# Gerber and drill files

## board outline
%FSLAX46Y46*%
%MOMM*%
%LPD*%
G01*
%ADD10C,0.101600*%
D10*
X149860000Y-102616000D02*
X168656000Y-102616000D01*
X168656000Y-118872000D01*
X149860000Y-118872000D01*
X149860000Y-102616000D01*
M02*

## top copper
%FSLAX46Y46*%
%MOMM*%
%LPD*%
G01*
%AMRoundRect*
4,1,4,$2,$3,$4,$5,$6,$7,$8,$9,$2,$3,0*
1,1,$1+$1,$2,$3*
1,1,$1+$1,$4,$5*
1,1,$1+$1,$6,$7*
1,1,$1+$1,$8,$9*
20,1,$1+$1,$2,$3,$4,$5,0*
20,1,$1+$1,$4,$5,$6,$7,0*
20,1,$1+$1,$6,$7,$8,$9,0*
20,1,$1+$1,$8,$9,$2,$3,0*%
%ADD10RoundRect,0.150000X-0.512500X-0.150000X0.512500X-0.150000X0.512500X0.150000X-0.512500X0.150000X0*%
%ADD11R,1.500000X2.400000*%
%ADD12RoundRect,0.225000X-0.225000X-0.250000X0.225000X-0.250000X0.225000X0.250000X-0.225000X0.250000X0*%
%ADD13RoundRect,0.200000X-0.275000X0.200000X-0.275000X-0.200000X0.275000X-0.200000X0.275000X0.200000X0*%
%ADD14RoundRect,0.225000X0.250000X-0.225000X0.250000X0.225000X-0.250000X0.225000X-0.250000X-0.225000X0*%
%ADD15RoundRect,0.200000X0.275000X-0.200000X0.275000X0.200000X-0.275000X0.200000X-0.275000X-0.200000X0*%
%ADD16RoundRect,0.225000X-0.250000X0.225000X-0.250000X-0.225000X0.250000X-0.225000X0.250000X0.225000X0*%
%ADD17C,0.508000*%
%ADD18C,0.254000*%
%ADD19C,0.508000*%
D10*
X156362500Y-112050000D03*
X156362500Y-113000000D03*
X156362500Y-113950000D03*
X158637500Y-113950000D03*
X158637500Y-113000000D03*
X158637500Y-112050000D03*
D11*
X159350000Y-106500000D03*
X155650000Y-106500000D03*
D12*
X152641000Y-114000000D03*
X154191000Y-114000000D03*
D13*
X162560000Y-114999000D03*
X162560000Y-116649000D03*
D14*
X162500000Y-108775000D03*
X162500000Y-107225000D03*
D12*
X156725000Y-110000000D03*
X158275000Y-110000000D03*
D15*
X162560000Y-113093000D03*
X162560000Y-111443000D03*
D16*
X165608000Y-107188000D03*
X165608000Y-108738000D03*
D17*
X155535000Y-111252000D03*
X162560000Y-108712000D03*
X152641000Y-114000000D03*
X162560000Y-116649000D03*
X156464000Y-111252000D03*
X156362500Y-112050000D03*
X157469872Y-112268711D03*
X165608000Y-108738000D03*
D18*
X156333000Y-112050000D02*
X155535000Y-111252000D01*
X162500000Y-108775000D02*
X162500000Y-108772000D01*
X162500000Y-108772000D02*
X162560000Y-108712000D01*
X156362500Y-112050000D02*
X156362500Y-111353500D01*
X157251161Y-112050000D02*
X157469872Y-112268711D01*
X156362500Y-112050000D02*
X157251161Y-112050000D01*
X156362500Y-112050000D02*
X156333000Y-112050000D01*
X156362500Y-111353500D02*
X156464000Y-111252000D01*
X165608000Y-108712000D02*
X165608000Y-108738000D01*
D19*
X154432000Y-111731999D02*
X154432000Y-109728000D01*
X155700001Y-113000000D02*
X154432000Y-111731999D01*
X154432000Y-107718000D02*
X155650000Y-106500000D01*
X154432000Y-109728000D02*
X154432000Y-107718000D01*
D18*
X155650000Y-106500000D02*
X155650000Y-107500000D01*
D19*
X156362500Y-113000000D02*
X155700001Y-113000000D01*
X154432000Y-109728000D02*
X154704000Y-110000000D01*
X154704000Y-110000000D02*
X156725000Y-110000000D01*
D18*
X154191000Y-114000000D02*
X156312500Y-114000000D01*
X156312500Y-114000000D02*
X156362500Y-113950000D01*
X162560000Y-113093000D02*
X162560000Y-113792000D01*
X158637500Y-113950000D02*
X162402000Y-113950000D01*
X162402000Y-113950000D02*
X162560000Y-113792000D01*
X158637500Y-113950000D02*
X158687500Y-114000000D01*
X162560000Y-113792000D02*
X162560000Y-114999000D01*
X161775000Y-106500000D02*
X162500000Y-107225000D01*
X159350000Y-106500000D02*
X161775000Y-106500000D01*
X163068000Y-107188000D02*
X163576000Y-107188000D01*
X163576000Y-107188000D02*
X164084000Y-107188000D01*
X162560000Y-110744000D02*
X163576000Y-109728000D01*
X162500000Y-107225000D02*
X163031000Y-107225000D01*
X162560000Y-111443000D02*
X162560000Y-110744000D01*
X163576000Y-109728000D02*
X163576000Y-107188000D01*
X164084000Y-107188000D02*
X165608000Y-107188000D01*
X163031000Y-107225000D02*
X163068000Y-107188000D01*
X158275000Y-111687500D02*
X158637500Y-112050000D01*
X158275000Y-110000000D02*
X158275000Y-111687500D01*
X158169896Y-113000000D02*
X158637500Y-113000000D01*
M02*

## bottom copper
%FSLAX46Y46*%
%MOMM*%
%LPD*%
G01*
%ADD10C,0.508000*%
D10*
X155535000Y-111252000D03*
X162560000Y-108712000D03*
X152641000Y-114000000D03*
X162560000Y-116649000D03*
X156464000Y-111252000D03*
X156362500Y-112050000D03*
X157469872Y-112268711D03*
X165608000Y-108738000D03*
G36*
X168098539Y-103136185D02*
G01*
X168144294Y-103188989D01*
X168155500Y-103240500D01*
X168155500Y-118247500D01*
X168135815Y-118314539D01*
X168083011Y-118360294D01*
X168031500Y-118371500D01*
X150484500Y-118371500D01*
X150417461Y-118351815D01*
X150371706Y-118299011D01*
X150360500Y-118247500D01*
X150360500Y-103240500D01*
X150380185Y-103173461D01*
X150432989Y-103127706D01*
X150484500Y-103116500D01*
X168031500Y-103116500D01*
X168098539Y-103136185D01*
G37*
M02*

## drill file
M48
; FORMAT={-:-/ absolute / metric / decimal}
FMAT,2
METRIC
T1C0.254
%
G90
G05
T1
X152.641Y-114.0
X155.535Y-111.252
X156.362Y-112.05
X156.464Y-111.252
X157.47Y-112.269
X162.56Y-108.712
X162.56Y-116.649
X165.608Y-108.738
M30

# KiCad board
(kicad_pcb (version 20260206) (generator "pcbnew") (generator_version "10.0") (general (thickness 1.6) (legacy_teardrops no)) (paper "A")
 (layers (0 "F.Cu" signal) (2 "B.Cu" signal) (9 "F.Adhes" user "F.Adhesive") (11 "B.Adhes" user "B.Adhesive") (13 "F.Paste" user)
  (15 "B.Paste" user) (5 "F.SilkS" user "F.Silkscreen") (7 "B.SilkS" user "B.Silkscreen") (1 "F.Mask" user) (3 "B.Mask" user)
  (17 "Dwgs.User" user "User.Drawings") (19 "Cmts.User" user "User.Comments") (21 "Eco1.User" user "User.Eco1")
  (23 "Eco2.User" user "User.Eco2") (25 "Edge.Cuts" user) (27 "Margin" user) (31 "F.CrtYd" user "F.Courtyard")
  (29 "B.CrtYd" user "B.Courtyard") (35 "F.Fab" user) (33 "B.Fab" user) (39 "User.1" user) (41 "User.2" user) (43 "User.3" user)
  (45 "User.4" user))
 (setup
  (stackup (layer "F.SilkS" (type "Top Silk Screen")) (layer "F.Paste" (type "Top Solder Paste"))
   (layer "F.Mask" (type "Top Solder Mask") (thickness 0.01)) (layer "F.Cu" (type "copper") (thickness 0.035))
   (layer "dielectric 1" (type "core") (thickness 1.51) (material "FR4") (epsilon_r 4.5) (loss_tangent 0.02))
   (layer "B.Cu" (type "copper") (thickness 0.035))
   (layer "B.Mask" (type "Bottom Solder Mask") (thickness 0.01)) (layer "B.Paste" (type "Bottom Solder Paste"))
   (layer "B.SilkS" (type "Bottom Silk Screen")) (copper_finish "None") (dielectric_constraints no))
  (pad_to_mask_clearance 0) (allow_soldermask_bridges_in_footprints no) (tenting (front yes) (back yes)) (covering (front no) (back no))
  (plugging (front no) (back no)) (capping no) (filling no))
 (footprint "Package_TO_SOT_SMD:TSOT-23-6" (layer "F.Cu") (at 157.5 113)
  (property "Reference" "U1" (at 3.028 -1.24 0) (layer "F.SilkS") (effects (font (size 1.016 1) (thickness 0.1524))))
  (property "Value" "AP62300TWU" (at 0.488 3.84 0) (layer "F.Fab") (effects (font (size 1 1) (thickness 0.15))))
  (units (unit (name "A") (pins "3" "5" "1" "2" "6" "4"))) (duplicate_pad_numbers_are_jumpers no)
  (pad "1" smd roundrect (at -1.1375 -0.95) (size 1.325 0.6) (layers "F.Cu" "F.Mask" "F.Paste") (roundrect_rratio 0.25) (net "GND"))
  (pad "2" smd roundrect (at -1.1375 0) (size 1.325 0.6) (layers "F.Cu" "F.Mask" "F.Paste") (roundrect_rratio 0.25) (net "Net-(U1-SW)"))
  (pad "3" smd roundrect (at -1.1375 0.95) (size 1.325 0.6) (layers "F.Cu" "F.Mask" "F.Paste") (roundrect_rratio 0.25) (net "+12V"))
  (pad "4" smd roundrect (at 1.1375 0.95) (size 1.325 0.6) (layers "F.Cu" "F.Mask" "F.Paste") (roundrect_rratio 0.25) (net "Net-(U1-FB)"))
  (pad "5" smd roundrect (at 1.1375 0) (size 1.325 0.6) (layers "F.Cu" "F.Mask" "F.Paste") (roundrect_rratio 0.25)
   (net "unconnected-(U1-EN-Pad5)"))
  (pad "6" smd roundrect (at 1.1375 -0.95) (size 1.325 0.6) (layers "F.Cu" "F.Mask" "F.Paste") (roundrect_rratio 0.25) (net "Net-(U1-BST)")))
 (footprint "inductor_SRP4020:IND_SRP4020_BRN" (layer "F.Cu") (at 157.5 106.5 180)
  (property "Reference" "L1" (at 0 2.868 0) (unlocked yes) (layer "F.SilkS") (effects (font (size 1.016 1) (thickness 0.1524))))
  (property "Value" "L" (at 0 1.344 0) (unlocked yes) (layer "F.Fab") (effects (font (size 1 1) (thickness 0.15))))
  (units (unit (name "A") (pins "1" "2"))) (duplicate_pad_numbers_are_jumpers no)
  (pad "1" smd rect (at -1.85 0 270) (size 2.4 1.5) (layers "F.Cu" "F.Mask" "F.Paste") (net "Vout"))
  (pad "2" smd rect (at 1.85 0 270) (size 2.4 1.5) (layers "F.Cu" "F.Mask" "F.Paste") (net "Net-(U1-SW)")))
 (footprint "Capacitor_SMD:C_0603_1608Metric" (layer "F.Cu") (at 153.416 114)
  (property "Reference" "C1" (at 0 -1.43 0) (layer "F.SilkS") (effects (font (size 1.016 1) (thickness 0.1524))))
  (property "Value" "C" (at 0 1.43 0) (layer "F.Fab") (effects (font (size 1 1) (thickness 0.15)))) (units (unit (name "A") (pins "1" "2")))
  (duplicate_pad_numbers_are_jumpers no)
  (pad "1" smd roundrect (at -0.775 0) (size 0.9 0.95) (layers "F.Cu" "F.Mask" "F.Paste") (roundrect_rratio 0.25) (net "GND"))
  (pad "2" smd roundrect (at 0.775 0) (size 0.9 0.95) (layers "F.Cu" "F.Mask" "F.Paste") (roundrect_rratio 0.25) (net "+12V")))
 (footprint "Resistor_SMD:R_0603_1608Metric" (layer "F.Cu") (at 162.56 115.824 -90)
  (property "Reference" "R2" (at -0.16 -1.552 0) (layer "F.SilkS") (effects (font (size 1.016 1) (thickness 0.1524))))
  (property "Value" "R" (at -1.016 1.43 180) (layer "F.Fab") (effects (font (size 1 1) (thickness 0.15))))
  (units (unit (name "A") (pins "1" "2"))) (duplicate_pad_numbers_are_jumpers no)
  (pad "1" smd roundrect (at -0.825 0 270) (size 0.8 0.95) (layers "F.Cu" "F.Mask" "F.Paste") (roundrect_rratio 0.25) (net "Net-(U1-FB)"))
  (pad "2" smd roundrect (at 0.825 0 270) (size 0.8 0.95) (layers "F.Cu" "F.Mask" "F.Paste") (roundrect_rratio 0.25) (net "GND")))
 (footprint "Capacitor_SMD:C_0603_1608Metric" (layer "F.Cu") (at 162.5 108 90)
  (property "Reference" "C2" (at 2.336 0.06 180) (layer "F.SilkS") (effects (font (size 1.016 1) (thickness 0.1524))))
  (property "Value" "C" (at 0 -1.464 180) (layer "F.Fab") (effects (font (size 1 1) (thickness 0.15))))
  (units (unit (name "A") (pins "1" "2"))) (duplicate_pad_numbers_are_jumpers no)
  (pad "1" smd roundrect (at -0.775 0 90) (size 0.9 0.95) (layers "F.Cu" "F.Mask" "F.Paste") (roundrect_rratio 0.25) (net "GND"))
  (pad "2" smd roundrect (at 0.775 0 90) (size 0.9 0.95) (layers "F.Cu" "F.Mask" "F.Paste") (roundrect_rratio 0.25) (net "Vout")))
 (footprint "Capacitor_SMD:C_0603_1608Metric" (layer "F.Cu") (at 157.5 110)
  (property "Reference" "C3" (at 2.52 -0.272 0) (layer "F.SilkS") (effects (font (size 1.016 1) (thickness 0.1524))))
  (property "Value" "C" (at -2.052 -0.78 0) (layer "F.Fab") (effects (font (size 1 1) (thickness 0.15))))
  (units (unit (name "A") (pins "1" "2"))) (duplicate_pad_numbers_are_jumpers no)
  (pad "1" smd roundrect (at -0.775 0) (size 0.9 0.95) (layers "F.Cu" "F.Mask" "F.Paste") (roundrect_rratio 0.25) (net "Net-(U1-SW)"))
  (pad "2" smd roundrect (at 0.775 0) (size 0.9 0.95) (layers "F.Cu" "F.Mask" "F.Paste") (roundrect_rratio 0.25) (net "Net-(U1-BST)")))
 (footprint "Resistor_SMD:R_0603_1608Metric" (layer "F.Cu") (at 162.56 112.268 90)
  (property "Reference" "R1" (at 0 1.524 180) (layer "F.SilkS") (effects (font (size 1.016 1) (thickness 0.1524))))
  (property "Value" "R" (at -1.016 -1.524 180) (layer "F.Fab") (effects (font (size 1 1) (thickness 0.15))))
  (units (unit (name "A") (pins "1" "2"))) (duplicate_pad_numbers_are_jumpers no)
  (pad "1" smd roundrect (at -0.825 0 90) (size 0.8 0.95) (layers "F.Cu" "F.Mask" "F.Paste") (roundrect_rratio 0.25) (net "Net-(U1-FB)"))
  (pad "2" smd roundrect (at 0.825 0 90) (size 0.8 0.95) (layers "F.Cu" "F.Mask" "F.Paste") (roundrect_rratio 0.25) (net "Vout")))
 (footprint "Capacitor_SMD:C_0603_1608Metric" (layer "F.Cu") (at 165.608 107.963 -90)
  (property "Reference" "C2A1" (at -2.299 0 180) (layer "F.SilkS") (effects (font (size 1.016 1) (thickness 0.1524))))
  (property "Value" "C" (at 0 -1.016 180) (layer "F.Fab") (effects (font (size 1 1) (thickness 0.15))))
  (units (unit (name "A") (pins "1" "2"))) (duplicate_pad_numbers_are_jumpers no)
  (pad "1" smd roundrect (at -0.775 0 270) (size 0.9 0.95) (layers "F.Cu" "F.Mask" "F.Paste") (roundrect_rratio 0.25) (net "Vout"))
  (pad "2" smd roundrect (at 0.775 0 270) (size 0.9 0.95) (layers "F.Cu" "F.Mask" "F.Paste") (roundrect_rratio 0.25) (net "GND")))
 (gr_rect (start 149.86 102.616) (end 168.656 118.872) (stroke (width 0.1016) (type default)) (fill no) (layer "Edge.Cuts"))
 (segment (start 156.333 112.05) (end 155.535 111.252) (width 0.254) (layer "F.Cu") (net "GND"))
 (segment (start 162.5 108.775) (end 162.5 108.772) (width 0.254) (layer "F.Cu") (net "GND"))
 (segment (start 162.5 108.772) (end 162.56 108.712) (width 0.254) (layer "F.Cu") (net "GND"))
 (segment (start 156.3625 112.05) (end 156.3625 111.3535) (width 0.254) (layer "F.Cu") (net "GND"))
 (segment (start 157.251161 112.05) (end 157.469872 112.268711) (width 0.254) (layer "F.Cu") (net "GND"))
 (segment (start 156.3625 112.05) (end 157.251161 112.05) (width 0.254) (layer "F.Cu") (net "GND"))
 (segment (start 156.3625 112.05) (end 156.333 112.05) (width 0.254) (layer "F.Cu") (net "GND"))
 (segment (start 156.3625 111.3535) (end 156.464 111.252) (width 0.254) (layer "F.Cu") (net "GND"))
 (segment (start 165.608 108.712) (end 165.608 108.738) (width 0.254) (layer "F.Cu") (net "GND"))
 (via (at 155.535 111.252) (size 0.508) (drill 0.254) (layers "F.Cu" "B.Cu") (free yes) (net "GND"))
 (via (at 162.56 108.712) (size 0.508) (drill 0.254) (layers "F.Cu" "B.Cu") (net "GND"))
 (via (at 152.641 114) (size 0.508) (drill 0.254) (layers "F.Cu" "B.Cu") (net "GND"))
 (via (at 162.56 116.649) (size 0.508) (drill 0.254) (layers "F.Cu" "B.Cu") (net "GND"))
 (via (at 156.464 111.252) (size 0.508) (drill 0.254) (layers "F.Cu" "B.Cu") (free yes) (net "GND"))
 (via (at 156.3625 112.05) (size 0.508) (drill 0.254) (layers "F.Cu" "B.Cu") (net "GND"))
 (via (at 157.469872 112.268711) (size 0.508) (drill 0.254) (layers "F.Cu" "B.Cu") (free yes) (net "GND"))
 (via (at 165.608 108.738) (size 0.508) (drill 0.254) (layers "F.Cu" "B.Cu") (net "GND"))
 (segment (start 154.432 111.731999) (end 154.432 109.728) (width 0.508) (layer "F.Cu") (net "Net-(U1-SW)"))
 (segment (start 155.700001 113) (end 154.432 111.731999) (width 0.508) (layer "F.Cu") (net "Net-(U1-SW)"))
 (segment (start 154.432 107.718) (end 155.65 106.5) (width 0.508) (layer "F.Cu") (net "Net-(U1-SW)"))
 (segment (start 154.432 109.728) (end 154.432 107.718) (width 0.508) (layer "F.Cu") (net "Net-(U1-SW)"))
 (segment (start 155.65 106.5) (end 155.65 107.5) (width 0.254) (layer "F.Cu") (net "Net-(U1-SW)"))
 (segment (start 156.3625 113) (end 155.700001 113) (width 0.508) (layer "F.Cu") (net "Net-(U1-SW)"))
 (segment (start 154.432 109.728) (end 154.704 110) (width 0.508) (layer "F.Cu") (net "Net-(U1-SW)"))
 (segment (start 154.704 110) (end 156.725 110) (width 0.508) (layer "F.Cu") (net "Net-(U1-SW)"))
 (segment (start 154.191 114) (end 156.3125 114) (width 0.254) (layer "F.Cu") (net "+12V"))
 (segment (start 156.3125 114) (end 156.3625 113.95) (width 0.254) (layer "F.Cu") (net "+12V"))
 (segment (start 162.56 113.093) (end 162.56 113.792) (width 0.254) (layer "F.Cu") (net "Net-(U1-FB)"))
 (segment (start 158.6375 113.95) (end 162.402 113.95) (width 0.254) (layer "F.Cu") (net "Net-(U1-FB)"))
 (segment (start 162.402 113.95) (end 162.56 113.792) (width 0.254) (layer "F.Cu") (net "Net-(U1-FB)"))
 (segment (start 158.6375 113.95) (end 158.6875 114) (width 0.254) (layer "F.Cu") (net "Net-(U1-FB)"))
 (segment (start 162.56 113.792) (end 162.56 114.999) (width 0.254) (layer "F.Cu") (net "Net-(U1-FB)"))
 (segment (start 161.775 106.5) (end 162.5 107.225) (width 0.254) (layer "F.Cu") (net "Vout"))
 (segment (start 159.35 106.5) (end 161.775 106.5) (width 0.254) (layer "F.Cu") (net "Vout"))
 (segment (start 163.068 107.188) (end 163.576 107.188) (width 0.254) (layer "F.Cu") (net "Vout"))
 (segment (start 163.576 107.188) (end 164.084 107.188) (width 0.254) (layer "F.Cu") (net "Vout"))
 (segment (start 162.56 110.744) (end 163.576 109.728) (width 0.254) (layer "F.Cu") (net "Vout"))
 (segment (start 162.5 107.225) (end 163.031 107.225) (width 0.254) (layer "F.Cu") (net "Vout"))
 (segment (start 162.56 111.443) (end 162.56 110.744) (width 0.254) (layer "F.Cu") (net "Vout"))
 (segment (start 163.576 109.728) (end 163.576 107.188) (width 0.254) (layer "F.Cu") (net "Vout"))
 (segment (start 164.084 107.188) (end 165.608 107.188) (width 0.254) (layer "F.Cu") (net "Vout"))
 (segment (start 163.031 107.225) (end 163.068 107.188) (width 0.254) (layer "F.Cu") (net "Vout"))
 (segment (start 158.275 111.6875) (end 158.6375 112.05) (width 0.254) (layer "F.Cu") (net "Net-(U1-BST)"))
 (segment (start 158.275 110) (end 158.275 111.6875) (width 0.254) (layer "F.Cu") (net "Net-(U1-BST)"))
 (segment (start 158.169896 113) (end 158.6375 113) (width 0.254) (layer "F.Cu") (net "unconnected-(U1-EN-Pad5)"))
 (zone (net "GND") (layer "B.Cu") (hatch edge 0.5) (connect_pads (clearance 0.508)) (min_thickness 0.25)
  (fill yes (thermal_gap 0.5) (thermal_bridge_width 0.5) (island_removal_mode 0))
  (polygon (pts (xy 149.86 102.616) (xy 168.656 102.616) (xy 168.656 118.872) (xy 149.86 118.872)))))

